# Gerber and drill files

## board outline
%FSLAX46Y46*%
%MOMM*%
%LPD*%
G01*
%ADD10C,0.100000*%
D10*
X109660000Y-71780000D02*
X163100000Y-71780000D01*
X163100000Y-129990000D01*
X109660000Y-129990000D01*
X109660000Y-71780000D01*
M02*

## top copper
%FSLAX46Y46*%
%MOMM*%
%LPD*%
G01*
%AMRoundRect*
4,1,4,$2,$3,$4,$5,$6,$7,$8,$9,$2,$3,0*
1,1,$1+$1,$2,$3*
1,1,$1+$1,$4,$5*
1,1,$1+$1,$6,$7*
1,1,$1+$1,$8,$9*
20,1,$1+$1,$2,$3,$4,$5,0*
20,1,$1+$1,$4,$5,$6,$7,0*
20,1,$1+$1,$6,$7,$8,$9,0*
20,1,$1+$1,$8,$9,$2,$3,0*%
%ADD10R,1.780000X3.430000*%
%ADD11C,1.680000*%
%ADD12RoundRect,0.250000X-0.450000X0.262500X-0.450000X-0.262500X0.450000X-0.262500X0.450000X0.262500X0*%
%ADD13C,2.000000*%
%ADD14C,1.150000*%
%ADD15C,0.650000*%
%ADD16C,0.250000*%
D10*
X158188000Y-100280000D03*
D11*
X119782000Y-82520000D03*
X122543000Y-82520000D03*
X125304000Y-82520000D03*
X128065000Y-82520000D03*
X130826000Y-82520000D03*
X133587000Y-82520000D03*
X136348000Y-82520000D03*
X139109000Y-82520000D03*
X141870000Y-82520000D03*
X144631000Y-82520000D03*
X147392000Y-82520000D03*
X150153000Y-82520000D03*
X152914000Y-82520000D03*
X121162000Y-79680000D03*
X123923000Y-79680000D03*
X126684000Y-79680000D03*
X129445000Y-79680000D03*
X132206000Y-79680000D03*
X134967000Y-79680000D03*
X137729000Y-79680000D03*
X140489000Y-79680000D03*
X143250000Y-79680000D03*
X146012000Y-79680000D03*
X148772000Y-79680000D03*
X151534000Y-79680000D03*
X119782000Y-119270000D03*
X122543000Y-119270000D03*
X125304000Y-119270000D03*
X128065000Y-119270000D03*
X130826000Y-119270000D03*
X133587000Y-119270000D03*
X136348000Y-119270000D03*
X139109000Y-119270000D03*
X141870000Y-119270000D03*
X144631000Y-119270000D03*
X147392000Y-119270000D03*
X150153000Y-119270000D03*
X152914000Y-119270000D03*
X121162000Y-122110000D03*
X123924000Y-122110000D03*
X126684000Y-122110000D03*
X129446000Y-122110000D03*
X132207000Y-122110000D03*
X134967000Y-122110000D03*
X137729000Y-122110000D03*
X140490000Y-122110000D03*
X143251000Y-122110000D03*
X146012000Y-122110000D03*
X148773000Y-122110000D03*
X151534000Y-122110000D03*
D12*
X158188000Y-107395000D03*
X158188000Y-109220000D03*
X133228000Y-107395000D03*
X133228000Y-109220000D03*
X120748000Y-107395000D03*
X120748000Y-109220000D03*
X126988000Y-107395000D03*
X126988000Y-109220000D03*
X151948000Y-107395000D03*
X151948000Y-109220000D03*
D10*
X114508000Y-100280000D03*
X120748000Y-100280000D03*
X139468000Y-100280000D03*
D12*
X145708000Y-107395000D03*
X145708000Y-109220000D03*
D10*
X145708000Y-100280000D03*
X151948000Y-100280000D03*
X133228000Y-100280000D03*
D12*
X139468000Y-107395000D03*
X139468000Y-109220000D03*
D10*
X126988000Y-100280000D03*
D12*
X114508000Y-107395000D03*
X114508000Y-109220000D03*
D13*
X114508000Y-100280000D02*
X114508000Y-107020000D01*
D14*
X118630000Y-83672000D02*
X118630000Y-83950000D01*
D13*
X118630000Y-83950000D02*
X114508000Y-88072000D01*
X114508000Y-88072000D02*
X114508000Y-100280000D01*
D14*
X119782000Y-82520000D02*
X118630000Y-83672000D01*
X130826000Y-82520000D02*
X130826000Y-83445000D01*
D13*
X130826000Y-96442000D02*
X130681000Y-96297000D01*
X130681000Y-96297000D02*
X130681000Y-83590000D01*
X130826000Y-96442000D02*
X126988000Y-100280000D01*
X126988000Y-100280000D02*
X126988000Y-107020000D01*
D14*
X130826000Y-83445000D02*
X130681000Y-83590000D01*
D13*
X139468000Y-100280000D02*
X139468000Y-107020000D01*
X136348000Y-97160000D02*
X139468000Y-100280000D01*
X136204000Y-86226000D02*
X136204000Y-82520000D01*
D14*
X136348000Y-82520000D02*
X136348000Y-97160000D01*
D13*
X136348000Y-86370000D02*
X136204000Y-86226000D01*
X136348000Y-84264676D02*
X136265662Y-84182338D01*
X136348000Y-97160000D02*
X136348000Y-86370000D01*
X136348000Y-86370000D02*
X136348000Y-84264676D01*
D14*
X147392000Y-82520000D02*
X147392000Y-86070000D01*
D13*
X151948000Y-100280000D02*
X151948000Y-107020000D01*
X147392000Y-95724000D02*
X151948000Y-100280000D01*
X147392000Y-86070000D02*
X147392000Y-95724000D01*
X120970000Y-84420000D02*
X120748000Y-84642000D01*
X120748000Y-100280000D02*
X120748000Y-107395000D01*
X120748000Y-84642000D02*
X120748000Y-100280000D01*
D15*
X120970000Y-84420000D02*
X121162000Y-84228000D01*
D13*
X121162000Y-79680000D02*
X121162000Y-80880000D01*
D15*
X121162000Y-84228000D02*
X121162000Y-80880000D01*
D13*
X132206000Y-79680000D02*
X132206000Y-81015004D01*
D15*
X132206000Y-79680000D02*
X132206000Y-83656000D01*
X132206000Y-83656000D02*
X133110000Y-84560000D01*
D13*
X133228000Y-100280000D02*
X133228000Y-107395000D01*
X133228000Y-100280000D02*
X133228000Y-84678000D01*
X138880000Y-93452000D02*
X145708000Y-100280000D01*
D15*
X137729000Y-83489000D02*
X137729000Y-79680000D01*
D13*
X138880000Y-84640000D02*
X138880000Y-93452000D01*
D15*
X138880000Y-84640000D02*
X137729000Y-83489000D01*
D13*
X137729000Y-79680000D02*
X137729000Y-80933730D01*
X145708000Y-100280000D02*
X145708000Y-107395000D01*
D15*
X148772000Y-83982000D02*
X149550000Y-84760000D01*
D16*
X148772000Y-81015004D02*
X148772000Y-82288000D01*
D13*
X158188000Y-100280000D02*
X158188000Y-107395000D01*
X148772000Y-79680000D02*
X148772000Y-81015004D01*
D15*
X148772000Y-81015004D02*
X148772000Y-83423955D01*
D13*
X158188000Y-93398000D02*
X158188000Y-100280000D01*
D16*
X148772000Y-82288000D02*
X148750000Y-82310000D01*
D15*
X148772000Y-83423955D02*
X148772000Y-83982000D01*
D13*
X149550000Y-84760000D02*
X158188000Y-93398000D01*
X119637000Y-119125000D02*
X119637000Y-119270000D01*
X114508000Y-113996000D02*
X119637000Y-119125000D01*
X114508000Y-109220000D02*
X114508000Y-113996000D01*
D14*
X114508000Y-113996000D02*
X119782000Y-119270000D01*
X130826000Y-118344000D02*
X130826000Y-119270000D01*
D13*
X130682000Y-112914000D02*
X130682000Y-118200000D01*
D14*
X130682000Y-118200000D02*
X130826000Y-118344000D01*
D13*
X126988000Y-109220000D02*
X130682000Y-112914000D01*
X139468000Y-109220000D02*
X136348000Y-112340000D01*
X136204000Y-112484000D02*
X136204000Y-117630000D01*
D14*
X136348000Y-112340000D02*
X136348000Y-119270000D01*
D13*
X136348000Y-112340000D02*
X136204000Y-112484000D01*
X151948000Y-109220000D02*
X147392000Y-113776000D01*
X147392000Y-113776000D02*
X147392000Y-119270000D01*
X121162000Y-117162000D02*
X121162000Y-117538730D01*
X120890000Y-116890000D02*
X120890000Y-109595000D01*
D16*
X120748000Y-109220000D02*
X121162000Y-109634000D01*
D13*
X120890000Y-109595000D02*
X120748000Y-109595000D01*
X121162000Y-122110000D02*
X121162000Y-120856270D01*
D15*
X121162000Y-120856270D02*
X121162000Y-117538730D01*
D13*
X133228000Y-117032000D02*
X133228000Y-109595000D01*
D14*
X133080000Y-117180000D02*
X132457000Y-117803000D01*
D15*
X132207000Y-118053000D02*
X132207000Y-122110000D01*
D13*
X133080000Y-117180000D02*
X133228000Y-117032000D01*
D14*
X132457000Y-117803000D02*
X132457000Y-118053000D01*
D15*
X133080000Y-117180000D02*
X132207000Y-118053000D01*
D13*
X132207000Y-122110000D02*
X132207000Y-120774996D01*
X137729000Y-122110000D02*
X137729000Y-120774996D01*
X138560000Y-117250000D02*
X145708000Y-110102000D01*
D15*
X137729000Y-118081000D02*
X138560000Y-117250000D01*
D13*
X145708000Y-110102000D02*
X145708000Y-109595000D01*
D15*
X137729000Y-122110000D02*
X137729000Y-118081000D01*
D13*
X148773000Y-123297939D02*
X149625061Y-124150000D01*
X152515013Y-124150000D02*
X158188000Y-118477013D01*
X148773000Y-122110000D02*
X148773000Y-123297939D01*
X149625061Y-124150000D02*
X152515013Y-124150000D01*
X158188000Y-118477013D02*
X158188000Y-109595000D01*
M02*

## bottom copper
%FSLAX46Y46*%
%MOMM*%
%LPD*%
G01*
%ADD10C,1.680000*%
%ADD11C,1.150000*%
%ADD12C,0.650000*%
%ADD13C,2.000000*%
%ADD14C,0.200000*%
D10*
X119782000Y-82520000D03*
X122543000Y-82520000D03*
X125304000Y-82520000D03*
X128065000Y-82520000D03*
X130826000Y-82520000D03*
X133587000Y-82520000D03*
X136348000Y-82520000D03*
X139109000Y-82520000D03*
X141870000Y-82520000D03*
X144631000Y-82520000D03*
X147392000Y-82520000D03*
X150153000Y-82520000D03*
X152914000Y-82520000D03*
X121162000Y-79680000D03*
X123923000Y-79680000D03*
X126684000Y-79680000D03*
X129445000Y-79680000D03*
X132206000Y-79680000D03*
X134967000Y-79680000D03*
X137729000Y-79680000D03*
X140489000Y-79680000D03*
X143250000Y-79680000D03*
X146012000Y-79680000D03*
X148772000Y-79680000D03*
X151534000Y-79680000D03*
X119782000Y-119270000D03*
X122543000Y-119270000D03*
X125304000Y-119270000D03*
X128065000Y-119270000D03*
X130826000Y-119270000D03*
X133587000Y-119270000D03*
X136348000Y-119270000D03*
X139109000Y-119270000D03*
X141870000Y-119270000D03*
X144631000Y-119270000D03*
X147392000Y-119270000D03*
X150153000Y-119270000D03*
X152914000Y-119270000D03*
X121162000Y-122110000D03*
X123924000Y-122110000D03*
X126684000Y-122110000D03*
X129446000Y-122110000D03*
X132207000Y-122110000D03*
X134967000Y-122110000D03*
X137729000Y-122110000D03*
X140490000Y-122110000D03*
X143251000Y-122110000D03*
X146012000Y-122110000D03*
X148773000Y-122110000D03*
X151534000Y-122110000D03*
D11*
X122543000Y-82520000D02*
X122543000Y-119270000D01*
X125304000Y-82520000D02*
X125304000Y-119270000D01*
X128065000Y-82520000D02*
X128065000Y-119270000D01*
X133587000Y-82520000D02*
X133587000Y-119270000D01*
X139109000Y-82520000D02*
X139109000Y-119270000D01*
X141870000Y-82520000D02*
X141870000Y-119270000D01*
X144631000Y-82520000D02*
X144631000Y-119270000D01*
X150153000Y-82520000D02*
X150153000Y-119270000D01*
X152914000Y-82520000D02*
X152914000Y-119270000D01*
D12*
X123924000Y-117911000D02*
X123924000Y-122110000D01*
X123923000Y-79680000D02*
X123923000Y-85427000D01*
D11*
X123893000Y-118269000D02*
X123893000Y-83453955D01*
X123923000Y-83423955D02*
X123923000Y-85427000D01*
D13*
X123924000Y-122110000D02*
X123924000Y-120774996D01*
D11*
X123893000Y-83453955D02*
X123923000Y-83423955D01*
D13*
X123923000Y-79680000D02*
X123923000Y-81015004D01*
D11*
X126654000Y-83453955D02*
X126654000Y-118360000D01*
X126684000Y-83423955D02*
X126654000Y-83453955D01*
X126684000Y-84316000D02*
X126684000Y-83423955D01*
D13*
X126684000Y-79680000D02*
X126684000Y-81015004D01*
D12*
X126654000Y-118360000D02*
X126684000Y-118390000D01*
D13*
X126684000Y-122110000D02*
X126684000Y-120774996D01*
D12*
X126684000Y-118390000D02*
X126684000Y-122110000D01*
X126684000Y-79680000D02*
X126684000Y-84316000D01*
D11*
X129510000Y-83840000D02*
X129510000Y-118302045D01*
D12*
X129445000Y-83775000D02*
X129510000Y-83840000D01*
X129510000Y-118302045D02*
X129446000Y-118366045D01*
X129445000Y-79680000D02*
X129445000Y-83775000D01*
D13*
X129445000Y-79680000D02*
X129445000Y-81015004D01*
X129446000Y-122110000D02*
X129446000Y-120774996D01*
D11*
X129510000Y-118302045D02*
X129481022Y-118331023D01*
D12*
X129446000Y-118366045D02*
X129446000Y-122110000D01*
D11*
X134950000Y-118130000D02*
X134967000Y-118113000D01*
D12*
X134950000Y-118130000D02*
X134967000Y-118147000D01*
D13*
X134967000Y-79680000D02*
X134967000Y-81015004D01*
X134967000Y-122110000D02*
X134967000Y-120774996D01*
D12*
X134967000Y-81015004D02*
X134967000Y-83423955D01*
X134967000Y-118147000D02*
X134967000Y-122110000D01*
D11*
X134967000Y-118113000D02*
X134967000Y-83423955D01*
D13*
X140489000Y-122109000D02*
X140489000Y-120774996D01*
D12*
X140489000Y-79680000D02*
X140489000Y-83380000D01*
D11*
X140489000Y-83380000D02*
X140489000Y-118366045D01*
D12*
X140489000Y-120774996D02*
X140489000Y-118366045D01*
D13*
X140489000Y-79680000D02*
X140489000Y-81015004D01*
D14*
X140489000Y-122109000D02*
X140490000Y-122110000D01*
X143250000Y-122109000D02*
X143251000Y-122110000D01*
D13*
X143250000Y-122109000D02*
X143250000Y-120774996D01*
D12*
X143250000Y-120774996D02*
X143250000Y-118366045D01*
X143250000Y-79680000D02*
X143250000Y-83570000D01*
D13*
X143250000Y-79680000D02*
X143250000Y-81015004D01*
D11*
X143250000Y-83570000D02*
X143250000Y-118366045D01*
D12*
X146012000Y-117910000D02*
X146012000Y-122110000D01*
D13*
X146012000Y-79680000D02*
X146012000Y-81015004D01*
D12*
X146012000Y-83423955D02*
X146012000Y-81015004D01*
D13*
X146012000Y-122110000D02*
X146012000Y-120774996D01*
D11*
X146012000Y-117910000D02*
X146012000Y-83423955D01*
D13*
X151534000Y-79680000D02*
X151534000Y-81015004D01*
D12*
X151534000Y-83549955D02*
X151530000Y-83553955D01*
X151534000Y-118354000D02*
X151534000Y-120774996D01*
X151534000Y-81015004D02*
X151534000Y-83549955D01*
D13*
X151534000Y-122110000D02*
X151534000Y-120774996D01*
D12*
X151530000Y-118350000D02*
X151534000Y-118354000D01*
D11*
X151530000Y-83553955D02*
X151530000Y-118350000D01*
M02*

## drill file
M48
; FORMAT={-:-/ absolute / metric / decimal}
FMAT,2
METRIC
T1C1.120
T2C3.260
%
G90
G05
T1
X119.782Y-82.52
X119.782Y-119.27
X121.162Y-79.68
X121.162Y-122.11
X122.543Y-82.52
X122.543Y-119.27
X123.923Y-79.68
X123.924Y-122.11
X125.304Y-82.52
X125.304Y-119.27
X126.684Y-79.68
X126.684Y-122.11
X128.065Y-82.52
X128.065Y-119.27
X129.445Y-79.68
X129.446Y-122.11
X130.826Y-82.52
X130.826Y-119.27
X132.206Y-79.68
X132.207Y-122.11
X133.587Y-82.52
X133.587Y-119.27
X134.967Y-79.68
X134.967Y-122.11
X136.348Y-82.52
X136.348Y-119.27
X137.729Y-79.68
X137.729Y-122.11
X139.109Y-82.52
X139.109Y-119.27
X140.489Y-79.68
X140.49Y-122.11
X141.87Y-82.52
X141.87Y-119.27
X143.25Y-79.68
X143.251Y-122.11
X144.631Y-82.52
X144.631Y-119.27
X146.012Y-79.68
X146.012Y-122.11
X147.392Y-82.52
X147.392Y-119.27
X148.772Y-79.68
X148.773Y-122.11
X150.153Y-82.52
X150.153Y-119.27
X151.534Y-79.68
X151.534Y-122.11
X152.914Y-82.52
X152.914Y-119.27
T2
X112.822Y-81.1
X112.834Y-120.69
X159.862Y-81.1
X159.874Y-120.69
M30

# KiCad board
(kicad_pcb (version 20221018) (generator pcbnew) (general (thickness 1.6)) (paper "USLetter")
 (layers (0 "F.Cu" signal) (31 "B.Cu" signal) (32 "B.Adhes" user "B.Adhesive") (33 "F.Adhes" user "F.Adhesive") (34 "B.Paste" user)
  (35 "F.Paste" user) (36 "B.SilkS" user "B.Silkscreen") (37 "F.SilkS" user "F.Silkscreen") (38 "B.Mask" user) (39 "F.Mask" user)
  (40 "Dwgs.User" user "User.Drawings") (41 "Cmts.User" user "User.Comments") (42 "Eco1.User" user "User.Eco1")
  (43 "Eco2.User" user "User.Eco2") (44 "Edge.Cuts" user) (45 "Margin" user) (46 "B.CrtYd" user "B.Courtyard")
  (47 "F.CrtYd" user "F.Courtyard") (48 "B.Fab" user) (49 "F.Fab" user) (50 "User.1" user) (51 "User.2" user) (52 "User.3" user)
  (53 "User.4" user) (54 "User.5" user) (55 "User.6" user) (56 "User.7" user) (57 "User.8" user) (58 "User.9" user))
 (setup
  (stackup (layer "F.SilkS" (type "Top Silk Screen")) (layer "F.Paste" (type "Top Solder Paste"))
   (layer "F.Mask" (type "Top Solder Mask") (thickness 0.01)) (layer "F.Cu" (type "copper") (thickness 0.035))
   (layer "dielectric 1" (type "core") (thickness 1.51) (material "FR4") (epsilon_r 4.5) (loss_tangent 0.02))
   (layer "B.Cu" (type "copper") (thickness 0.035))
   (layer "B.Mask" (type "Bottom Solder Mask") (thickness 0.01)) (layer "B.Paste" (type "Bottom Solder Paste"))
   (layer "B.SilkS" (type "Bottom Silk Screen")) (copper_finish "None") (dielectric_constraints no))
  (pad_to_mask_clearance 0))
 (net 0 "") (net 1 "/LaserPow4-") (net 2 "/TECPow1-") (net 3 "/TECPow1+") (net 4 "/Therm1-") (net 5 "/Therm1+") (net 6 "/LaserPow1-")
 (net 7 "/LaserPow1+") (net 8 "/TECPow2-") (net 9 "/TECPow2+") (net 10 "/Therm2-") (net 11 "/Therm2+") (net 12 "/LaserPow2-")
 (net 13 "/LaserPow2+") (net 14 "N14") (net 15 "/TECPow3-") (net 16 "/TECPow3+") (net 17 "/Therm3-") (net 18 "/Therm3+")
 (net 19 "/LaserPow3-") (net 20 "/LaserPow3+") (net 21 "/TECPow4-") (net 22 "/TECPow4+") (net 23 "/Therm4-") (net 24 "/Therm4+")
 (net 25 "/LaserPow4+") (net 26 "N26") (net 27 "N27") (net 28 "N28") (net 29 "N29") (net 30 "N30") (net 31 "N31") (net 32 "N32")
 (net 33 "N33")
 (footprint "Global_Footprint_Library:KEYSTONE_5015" (layer "F.Cu") (at 158.188 100.28 90)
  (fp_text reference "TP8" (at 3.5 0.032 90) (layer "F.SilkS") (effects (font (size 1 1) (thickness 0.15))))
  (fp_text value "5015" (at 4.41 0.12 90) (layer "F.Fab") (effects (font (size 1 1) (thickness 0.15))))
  (pad "TP" smd rect (at 0 0 90) (size 3.43 1.78) (layers "F.Cu" "F.Paste" "F.Mask") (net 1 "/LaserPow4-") (solder_mask_margin 0.102)))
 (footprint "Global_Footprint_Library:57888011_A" (layer "F.Cu") (at 119.782 82.52)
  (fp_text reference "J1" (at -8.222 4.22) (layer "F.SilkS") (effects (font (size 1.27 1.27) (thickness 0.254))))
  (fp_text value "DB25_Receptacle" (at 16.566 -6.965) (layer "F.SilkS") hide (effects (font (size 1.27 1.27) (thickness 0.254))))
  (pad "" np_thru_hole circle (at -6.96 -1.42) (size 3.26 3.26) (drill 3.26) (layers "*.Cu" "*.Mask"))
  (pad "" np_thru_hole circle (at 40.08 -1.42) (size 3.26 3.26) (drill 3.26) (layers "*.Cu" "*.Mask"))
  (pad "1" thru_hole circle (at 0 0) (size 1.68 1.68) (drill 1.12) (layers "*.Cu" "*.Mask") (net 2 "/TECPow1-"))
  (pad "2" thru_hole circle (at 2.761 0) (size 1.68 1.68) (drill 1.12) (layers "*.Cu" "*.Mask") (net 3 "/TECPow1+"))
  (pad "3" thru_hole circle (at 5.522 0) (size 1.68 1.68) (drill 1.12) (layers "*.Cu" "*.Mask") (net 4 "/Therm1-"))
  (pad "4" thru_hole circle (at 8.283 0) (size 1.68 1.68) (drill 1.12) (layers "*.Cu" "*.Mask") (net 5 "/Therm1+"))
  (pad "5" thru_hole circle (at 11.044 0) (size 1.68 1.68) (drill 1.12) (layers "*.Cu" "*.Mask") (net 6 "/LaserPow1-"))
  (pad "6" thru_hole circle (at 13.805 0) (size 1.68 1.68) (drill 1.12) (layers "*.Cu" "*.Mask") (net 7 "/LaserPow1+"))
  (pad "7" thru_hole circle (at 16.566 0) (size 1.68 1.68) (drill 1.12) (layers "*.Cu" "*.Mask") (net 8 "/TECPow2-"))
  (pad "8" thru_hole circle (at 19.327 0) (size 1.68 1.68) (drill 1.12) (layers "*.Cu" "*.Mask") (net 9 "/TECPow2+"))
  (pad "9" thru_hole circle (at 22.088 0) (size 1.68 1.68) (drill 1.12) (layers "*.Cu" "*.Mask") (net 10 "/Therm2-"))
  (pad "10" thru_hole circle (at 24.849 0) (size 1.68 1.68) (drill 1.12) (layers "*.Cu" "*.Mask") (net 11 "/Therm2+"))
  (pad "11" thru_hole circle (at 27.61 0) (size 1.68 1.68) (drill 1.12) (layers "*.Cu" "*.Mask") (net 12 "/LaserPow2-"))
  (pad "12" thru_hole circle (at 30.371 0) (size 1.68 1.68) (drill 1.12) (layers "*.Cu" "*.Mask") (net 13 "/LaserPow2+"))
  (pad "13" thru_hole circle (at 33.132 0) (size 1.68 1.68) (drill 1.12) (layers "*.Cu" "*.Mask") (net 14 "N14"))
  (pad "14" thru_hole circle (at 1.38 -2.84) (size 1.68 1.68) (drill 1.12) (layers "*.Cu" "*.Mask") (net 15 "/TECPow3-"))
  (pad "15" thru_hole circle (at 4.141 -2.84) (size 1.68 1.68) (drill 1.12) (layers "*.Cu" "*.Mask") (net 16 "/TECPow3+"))
  (pad "16" thru_hole circle (at 6.902 -2.84) (size 1.68 1.68) (drill 1.12) (layers "*.Cu" "*.Mask") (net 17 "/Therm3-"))
  (pad "17" thru_hole circle (at 9.663 -2.84) (size 1.68 1.68) (drill 1.12) (layers "*.Cu" "*.Mask") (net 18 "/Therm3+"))
  (pad "18" thru_hole circle (at 12.424 -2.84) (size 1.68 1.68) (drill 1.12) (layers "*.Cu" "*.Mask") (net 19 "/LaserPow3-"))
  (pad "19" thru_hole circle (at 15.185 -2.84) (size 1.68 1.68) (drill 1.12) (layers "*.Cu" "*.Mask") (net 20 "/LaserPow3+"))
  (pad "20" thru_hole circle (at 17.947 -2.84) (size 1.68 1.68) (drill 1.12) (layers "*.Cu" "*.Mask") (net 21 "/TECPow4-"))
  (pad "21" thru_hole circle (at 20.707 -2.84) (size 1.68 1.68) (drill 1.12) (layers "*.Cu" "*.Mask") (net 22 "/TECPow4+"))
  (pad "22" thru_hole circle (at 23.468 -2.84) (size 1.68 1.68) (drill 1.12) (layers "*.Cu" "*.Mask") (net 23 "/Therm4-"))
  (pad "23" thru_hole circle (at 26.23 -2.84) (size 1.68 1.68) (drill 1.12) (layers "*.Cu" "*.Mask") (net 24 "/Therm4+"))
  (pad "24" thru_hole circle (at 28.99 -2.84) (size 1.68 1.68) (drill 1.12) (layers "*.Cu" "*.Mask") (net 1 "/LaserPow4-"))
  (pad "25" thru_hole circle (at 31.752 -2.84) (size 1.68 1.68) (drill 1.12) (layers "*.Cu" "*.Mask") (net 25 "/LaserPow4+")))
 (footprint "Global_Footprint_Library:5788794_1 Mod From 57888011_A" (layer "F.Cu") (at 152.914 119.27 180)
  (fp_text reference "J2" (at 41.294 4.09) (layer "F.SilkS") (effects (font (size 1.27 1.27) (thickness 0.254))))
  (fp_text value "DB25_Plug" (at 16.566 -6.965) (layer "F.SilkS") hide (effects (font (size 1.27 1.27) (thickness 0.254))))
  (pad "" np_thru_hole circle (at -6.96 -1.42 180) (size 3.26 3.26) (drill 3.26) (layers "*.Cu" "*.Mask"))
  (pad "" np_thru_hole circle (at 40.08 -1.42 180) (size 3.26 3.26) (drill 3.26) (layers "*.Cu" "*.Mask"))
  (pad "1" thru_hole circle (at 33.132 0 180) (size 1.68 1.68) (drill 1.12) (layers "*.Cu" "*.Mask") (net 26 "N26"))
  (pad "2" thru_hole circle (at 30.371 0 180) (size 1.68 1.68) (drill 1.12) (layers "*.Cu" "*.Mask") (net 3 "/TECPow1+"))
  (pad "3" thru_hole circle (at 27.61 0 180) (size 1.68 1.68) (drill 1.12) (layers "*.Cu" "*.Mask") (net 4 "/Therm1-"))
  (pad "4" thru_hole circle (at 24.849 0 180) (size 1.68 1.68) (drill 1.12) (layers "*.Cu" "*.Mask") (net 5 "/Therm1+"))
  (pad "5" thru_hole circle (at 22.088 0 180) (size 1.68 1.68) (drill 1.12) (layers "*.Cu" "*.Mask") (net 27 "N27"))
  (pad "6" thru_hole circle (at 19.327 0 180) (size 1.68 1.68) (drill 1.12) (layers "*.Cu" "*.Mask") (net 7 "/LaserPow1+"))
  (pad "7" thru_hole circle (at 16.566 0 180) (size 1.68 1.68) (drill 1.12) (layers "*.Cu" "*.Mask") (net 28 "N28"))
  (pad "8" thru_hole circle (at 13.805 0 180) (size 1.68 1.68) (drill 1.12) (layers "*.Cu" "*.Mask") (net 9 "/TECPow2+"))
  (pad "9" thru_hole circle (at 11.044 0 180) (size 1.68 1.68) (drill 1.12) (layers "*.Cu" "*.Mask") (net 10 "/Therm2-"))
  (pad "10" thru_hole circle (at 8.283 0 180) (size 1.68 1.68) (drill 1.12) (layers "*.Cu" "*.Mask") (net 11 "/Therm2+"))
  (pad "11" thru_hole circle (at 5.522 0 180) (size 1.68 1.68) (drill 1.12) (layers "*.Cu" "*.Mask") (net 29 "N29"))
  (pad "12" thru_hole circle (at 2.761 0 180) (size 1.68 1.68) (drill 1.12) (layers "*.Cu" "*.Mask") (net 13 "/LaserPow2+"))
  (pad "13" thru_hole circle (at 0 0 180) (size 1.68 1.68) (drill 1.12) (layers "*.Cu" "*.Mask") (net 14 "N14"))
  (pad "14" thru_hole circle (at 31.752 -2.84 180) (size 1.68 1.68) (drill 1.12) (layers "*.Cu" "*.Mask") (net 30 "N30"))
  (pad "15" thru_hole circle (at 28.99 -2.84 180) (size 1.68 1.68) (drill 1.12) (layers "*.Cu" "*.Mask") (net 16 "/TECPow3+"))
  (pad "16" thru_hole circle (at 26.23 -2.84 180) (size 1.68 1.68) (drill 1.12) (layers "*.Cu" "*.Mask") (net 17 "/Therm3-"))
  (pad "17" thru_hole circle (at 23.468 -2.84 180) (size 1.68 1.68) (drill 1.12) (layers "*.Cu" "*.Mask") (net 18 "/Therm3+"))
  (pad "18" thru_hole circle (at 20.707 -2.84 180) (size 1.68 1.68) (drill 1.12) (layers "*.Cu" "*.Mask") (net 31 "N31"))
  (pad "19" thru_hole circle (at 17.947 -2.84 180) (size 1.68 1.68) (drill 1.12) (layers "*.Cu" "*.Mask") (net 20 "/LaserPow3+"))
  (pad "20" thru_hole circle (at 15.185 -2.84 180) (size 1.68 1.68) (drill 1.12) (layers "*.Cu" "*.Mask") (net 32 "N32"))
  (pad "21" thru_hole circle (at 12.424 -2.84 180) (size 1.68 1.68) (drill 1.12) (layers "*.Cu" "*.Mask") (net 22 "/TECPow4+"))
  (pad "22" thru_hole circle (at 9.663 -2.84 180) (size 1.68 1.68) (drill 1.12) (layers "*.Cu" "*.Mask") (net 23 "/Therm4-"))
  (pad "23" thru_hole circle (at 6.902 -2.84 180) (size 1.68 1.68) (drill 1.12) (layers "*.Cu" "*.Mask") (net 24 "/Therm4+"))
  (pad "24" thru_hole circle (at 4.141 -2.84 180) (size 1.68 1.68) (drill 1.12) (layers "*.Cu" "*.Mask") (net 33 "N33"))
  (pad "25" thru_hole circle (at 1.38 -2.84 180) (size 1.68 1.68) (drill 1.12) (layers "*.Cu" "*.Mask") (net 25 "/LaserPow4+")))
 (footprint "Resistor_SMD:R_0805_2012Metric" (layer "F.Cu") (at 158.188 108.3075 -90)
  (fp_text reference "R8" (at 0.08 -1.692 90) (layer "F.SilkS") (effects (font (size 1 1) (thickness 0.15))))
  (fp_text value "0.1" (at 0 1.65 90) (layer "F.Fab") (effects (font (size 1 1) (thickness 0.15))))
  (pad "1" smd roundrect (at -0.9125 0 270) (size 1.025 1.4) (layers "F.Cu" "F.Paste" "F.Mask") (roundrect_rratio 0.243902439)
   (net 1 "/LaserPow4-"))
  (pad "2" smd roundrect (at 0.9125 0 270) (size 1.025 1.4) (layers "F.Cu" "F.Paste" "F.Mask") (roundrect_rratio 0.243902439) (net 33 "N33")))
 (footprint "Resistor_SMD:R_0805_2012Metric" (layer "F.Cu") (at 133.228 108.3075 -90)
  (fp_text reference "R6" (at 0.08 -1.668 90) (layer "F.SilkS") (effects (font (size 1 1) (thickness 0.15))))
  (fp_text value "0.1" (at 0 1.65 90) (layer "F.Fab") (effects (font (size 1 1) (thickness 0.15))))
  (pad "1" smd roundrect (at -0.9125 0 270) (size 1.025 1.4) (layers "F.Cu" "F.Paste" "F.Mask") (roundrect_rratio 0.243902439)
   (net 19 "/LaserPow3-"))
  (pad "2" smd roundrect (at 0.9125 0 270) (size 1.025 1.4) (layers "F.Cu" "F.Paste" "F.Mask") (roundrect_rratio 0.243902439) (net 31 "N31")))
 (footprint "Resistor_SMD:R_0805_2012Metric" (layer "F.Cu") (at 120.748 108.3075 -90)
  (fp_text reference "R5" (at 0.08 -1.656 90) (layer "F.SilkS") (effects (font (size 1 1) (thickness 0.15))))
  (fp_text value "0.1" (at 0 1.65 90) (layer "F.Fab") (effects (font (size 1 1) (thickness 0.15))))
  (pad "1" smd roundrect (at -0.9125 0 270) (size 1.025 1.4) (layers "F.Cu" "F.Paste" "F.Mask") (roundrect_rratio 0.243902439)
   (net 15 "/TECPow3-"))
  (pad "2" smd roundrect (at 0.9125 0 270) (size 1.025 1.4) (layers "F.Cu" "F.Paste" "F.Mask") (roundrect_rratio 0.243902439) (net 30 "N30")))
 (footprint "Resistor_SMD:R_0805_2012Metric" (layer "F.Cu") (at 126.988 108.3075 -90)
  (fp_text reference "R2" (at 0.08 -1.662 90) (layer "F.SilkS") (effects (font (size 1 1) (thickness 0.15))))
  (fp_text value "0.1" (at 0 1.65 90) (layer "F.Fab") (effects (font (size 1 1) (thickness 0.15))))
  (pad "1" smd roundrect (at -0.9125 0 270) (size 1.025 1.4) (layers "F.Cu" "F.Paste" "F.Mask") (roundrect_rratio 0.243902439)
   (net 6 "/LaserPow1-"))
  (pad "2" smd roundrect (at 0.9125 0 270) (size 1.025 1.4) (layers "F.Cu" "F.Paste" "F.Mask") (roundrect_rratio 0.243902439) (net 27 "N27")))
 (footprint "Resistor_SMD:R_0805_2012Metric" (layer "F.Cu") (at 151.948 108.3075 -90)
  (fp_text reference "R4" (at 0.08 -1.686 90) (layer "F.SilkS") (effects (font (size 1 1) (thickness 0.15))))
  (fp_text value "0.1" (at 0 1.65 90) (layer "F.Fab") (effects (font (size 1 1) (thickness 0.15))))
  (pad "1" smd roundrect (at -0.9125 0 270) (size 1.025 1.4) (layers "F.Cu" "F.Paste" "F.Mask") (roundrect_rratio 0.243902439)
   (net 12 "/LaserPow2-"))
  (pad "2" smd roundrect (at 0.9125 0 270) (size 1.025 1.4) (layers "F.Cu" "F.Paste" "F.Mask") (roundrect_rratio 0.243902439) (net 29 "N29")))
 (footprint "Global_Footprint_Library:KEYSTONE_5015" (layer "F.Cu") (at 114.508 100.28 90)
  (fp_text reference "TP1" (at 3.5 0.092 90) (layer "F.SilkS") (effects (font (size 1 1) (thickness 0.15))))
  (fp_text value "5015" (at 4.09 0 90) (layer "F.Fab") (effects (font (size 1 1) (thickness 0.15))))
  (pad "TP" smd rect (at 0 0 90) (size 3.43 1.78) (layers "F.Cu" "F.Paste" "F.Mask") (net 2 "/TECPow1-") (solder_mask_margin 0.102)))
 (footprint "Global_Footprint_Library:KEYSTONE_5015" (layer "F.Cu") (at 120.748 100.28 90)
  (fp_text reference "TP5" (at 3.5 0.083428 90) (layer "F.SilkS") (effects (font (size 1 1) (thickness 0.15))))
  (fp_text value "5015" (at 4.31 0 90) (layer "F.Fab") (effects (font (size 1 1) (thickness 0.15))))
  (pad "TP" smd rect (at 0 0 90) (size 3.43 1.78) (layers "F.Cu" "F.Paste" "F.Mask") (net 15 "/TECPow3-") (solder_mask_margin 0.102)))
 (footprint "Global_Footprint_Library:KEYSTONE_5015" (layer "F.Cu") (at 139.468 100.28 90)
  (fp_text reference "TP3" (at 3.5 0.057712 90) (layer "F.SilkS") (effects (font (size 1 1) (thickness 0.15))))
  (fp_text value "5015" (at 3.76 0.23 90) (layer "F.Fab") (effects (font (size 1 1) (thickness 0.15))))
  (pad "TP" smd rect (at 0 0 90) (size 3.43 1.78) (layers "F.Cu" "F.Paste" "F.Mask") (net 8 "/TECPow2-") (solder_mask_margin 0.102)))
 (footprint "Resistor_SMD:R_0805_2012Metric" (layer "F.Cu") (at 145.708 108.3075 -90)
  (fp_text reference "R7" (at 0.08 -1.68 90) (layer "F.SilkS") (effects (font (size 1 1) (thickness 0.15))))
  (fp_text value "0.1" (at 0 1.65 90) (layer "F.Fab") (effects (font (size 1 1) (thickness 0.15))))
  (pad "1" smd roundrect (at -0.9125 0 270) (size 1.025 1.4) (layers "F.Cu" "F.Paste" "F.Mask") (roundrect_rratio 0.243902439)
   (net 21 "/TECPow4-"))
  (pad "2" smd roundrect (at 0.9125 0 270) (size 1.025 1.4) (layers "F.Cu" "F.Paste" "F.Mask") (roundrect_rratio 0.243902439) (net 32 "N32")))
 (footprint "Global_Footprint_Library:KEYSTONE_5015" (layer "F.Cu") (at 145.708 100.28 90)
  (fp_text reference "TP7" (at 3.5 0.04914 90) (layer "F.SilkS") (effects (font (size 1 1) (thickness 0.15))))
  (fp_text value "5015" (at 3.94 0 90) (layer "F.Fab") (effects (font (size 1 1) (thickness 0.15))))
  (pad "TP" smd rect (at 0 0 90) (size 3.43 1.78) (layers "F.Cu" "F.Paste" "F.Mask") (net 21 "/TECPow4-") (solder_mask_margin 0.102)))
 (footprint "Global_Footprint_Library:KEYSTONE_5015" (layer "F.Cu") (at 151.948 100.28 90)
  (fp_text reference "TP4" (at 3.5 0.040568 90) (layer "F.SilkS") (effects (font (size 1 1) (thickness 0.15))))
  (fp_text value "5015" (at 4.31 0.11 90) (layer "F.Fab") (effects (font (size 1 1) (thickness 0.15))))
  (pad "TP" smd rect (at 0 0 90) (size 3.43 1.78) (layers "F.Cu" "F.Paste" "F.Mask") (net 12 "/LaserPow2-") (solder_mask_margin 0.102)))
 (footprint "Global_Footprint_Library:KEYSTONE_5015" (layer "F.Cu") (at 133.228 100.28 90)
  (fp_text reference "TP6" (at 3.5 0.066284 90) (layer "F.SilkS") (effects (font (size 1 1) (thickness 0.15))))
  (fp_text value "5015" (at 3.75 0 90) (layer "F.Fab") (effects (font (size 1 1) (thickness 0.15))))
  (pad "TP" smd rect (at 0 0 90) (size 3.43 1.78) (layers "F.Cu" "F.Paste" "F.Mask") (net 19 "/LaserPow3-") (solder_mask_margin 0.102)))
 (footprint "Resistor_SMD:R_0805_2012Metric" (layer "F.Cu") (at 139.468 108.3075 -90)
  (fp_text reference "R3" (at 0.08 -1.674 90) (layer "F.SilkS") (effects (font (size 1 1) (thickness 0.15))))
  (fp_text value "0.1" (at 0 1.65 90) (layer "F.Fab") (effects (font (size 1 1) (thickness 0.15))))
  (pad "1" smd roundrect (at -0.9125 0 270) (size 1.025 1.4) (layers "F.Cu" "F.Paste" "F.Mask") (roundrect_rratio 0.243902439)
   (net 8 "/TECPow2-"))
  (pad "2" smd roundrect (at 0.9125 0 270) (size 1.025 1.4) (layers "F.Cu" "F.Paste" "F.Mask") (roundrect_rratio 0.243902439) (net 28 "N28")))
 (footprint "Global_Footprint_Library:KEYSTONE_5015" (layer "F.Cu") (at 126.988 100.28 90)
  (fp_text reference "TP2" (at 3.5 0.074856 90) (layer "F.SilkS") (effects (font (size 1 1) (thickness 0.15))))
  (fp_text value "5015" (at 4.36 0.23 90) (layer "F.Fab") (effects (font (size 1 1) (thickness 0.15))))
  (pad "TP" smd rect (at 0 0 90) (size 3.43 1.78) (layers "F.Cu" "F.Paste" "F.Mask") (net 6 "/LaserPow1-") (solder_mask_margin 0.102)))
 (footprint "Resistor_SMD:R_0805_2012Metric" (layer "F.Cu") (at 114.508 108.3075 -90)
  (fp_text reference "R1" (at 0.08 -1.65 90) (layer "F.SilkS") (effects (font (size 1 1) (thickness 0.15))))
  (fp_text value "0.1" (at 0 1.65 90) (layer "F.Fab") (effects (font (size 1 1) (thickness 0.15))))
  (pad "1" smd roundrect (at -0.9125 0 270) (size 1.025 1.4) (layers "F.Cu" "F.Paste" "F.Mask") (roundrect_rratio 0.243902439)
   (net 2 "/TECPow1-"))
  (pad "2" smd roundrect (at 0.9125 0 270) (size 1.025 1.4) (layers "F.Cu" "F.Paste" "F.Mask") (roundrect_rratio 0.243902439) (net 26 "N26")))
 (gr_rect (start 109.66 71.78) (end 163.1 129.99) (stroke (width 0.1) (type default)) (fill none) (layer "Edge.Cuts"))
 (segment (start 114.508 100.28) (end 114.508 107.02) (width 2) (layer "F.Cu") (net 2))
 (segment (start 118.63 83.672) (end 118.63 83.95) (width 1.15) (layer "F.Cu") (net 2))
 (segment (start 118.63 83.95) (end 114.508 88.072) (width 2) (layer "F.Cu") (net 2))
 (segment (start 114.508 88.072) (end 114.508 100.28) (width 2) (layer "F.Cu") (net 2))
 (segment (start 119.782 82.52) (end 118.63 83.672) (width 1.15) (layer "F.Cu") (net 2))
 (segment (start 122.543 82.52) (end 122.543 119.27) (width 1.15) (layer "B.Cu") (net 3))
 (segment (start 125.304 82.52) (end 125.304 119.27) (width 1.15) (layer "B.Cu") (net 4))
 (segment (start 128.065 82.52) (end 128.065 119.27) (width 1.15) (layer "B.Cu") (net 5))
 (segment (start 130.826 82.52) (end 130.826 83.445) (width 1.15) (layer "F.Cu") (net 6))
 (segment (start 130.826 96.442) (end 130.681 96.297) (width 2) (layer "F.Cu") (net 6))
 (segment (start 130.681 96.297) (end 130.681 83.59) (width 2) (layer "F.Cu") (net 6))
 (segment (start 130.826 96.442) (end 126.988 100.28) (width 2) (layer "F.Cu") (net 6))
 (segment (start 126.988 100.28) (end 126.988 107.02) (width 2) (layer "F.Cu") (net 6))
 (segment (start 130.826 83.445) (end 130.681 83.59) (width 1.15) (layer "F.Cu") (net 6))
 (segment (start 133.587 82.52) (end 133.587 119.27) (width 1.15) (layer "B.Cu") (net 7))
 (segment (start 139.468 100.28) (end 139.468 107.02) (width 2) (layer "F.Cu") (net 8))
 (segment (start 136.348 97.16) (end 139.468 100.28) (width 2) (layer "F.Cu") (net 8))
 (segment (start 136.204 86.226) (end 136.204 82.52) (width 2) (layer "F.Cu") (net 8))
 (segment (start 136.348 82.52) (end 136.348 97.16) (width 1.15) (layer "F.Cu") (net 8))
 (segment (start 136.348 86.37) (end 136.204 86.226) (width 2) (layer "F.Cu") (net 8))
 (segment (start 136.348 84.264676) (end 136.265662 84.182338) (width 2) (layer "F.Cu") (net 8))
 (segment (start 136.348 97.16) (end 136.348 86.37) (width 2) (layer "F.Cu") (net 8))
 (segment (start 136.348 86.37) (end 136.348 84.264676) (width 2) (layer "F.Cu") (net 8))
 (segment (start 139.109 82.52) (end 139.109 119.27) (width 1.15) (layer "B.Cu") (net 9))
 (segment (start 141.87 82.52) (end 141.87 119.27) (width 1.15) (layer "B.Cu") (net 10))
 (segment (start 144.631 82.52) (end 144.631 119.27) (width 1.15) (layer "B.Cu") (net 11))
 (segment (start 147.392 82.52) (end 147.392 86.07) (width 1.15) (layer "F.Cu") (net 12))
 (segment (start 151.948 100.28) (end 151.948 107.02) (width 2) (layer "F.Cu") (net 12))
 (segment (start 147.392 95.724) (end 151.948 100.28) (width 2) (layer "F.Cu") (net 12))
 (segment (start 147.392 86.07) (end 147.392 95.724) (width 2) (layer "F.Cu") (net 12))
 (segment (start 150.153 82.52) (end 150.153 119.27) (width 1.15) (layer "B.Cu") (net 13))
 (segment (start 152.914 82.52) (end 152.914 119.27) (width 1.15) (layer "B.Cu") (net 14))
 (segment (start 120.97 84.42) (end 120.748 84.642) (width 2) (layer "F.Cu") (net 15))
 (segment (start 120.748 100.28) (end 120.748 107.395) (width 2) (layer "F.Cu") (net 15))
 (segment (start 120.748 84.642) (end 120.748 100.28) (width 2) (layer "F.Cu") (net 15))
 (segment (start 120.97 84.42) (end 121.162 84.228) (width 0.65) (layer "F.Cu") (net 15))
 (segment (start 121.162 79.68) (end 121.162 80.88) (width 2) (layer "F.Cu") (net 15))
 (segment (start 121.162 84.228) (end 121.162 80.88) (width 0.65) (layer "F.Cu") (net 15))
 (segment (start 123.924 117.911) (end 123.924 122.11) (width 0.65) (layer "B.Cu") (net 16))
 (segment (start 123.923 79.68) (end 123.923 85.427) (width 0.65) (layer "B.Cu") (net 16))
 (segment (start 123.893 118.269) (end 123.893 83.453955) (width 1.15) (layer "B.Cu") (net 16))
 (segment (start 123.923 83.423955) (end 123.923 85.427) (width 1.15) (layer "B.Cu") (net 16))
 (segment (start 123.924 122.11) (end 123.924 120.774996) (width 2) (layer "B.Cu") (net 16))
 (segment (start 123.893 83.453955) (end 123.923 83.423955) (width 1.15) (layer "B.Cu") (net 16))
 (segment (start 123.923 79.68) (end 123.923 81.015004) (width 2) (layer "B.Cu") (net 16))
 (segment (start 126.654 83.453955) (end 126.654 118.36) (width 1.15) (layer "B.Cu") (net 17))
 (segment (start 126.684 83.423955) (end 126.654 83.453955) (width 1.15) (layer "B.Cu") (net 17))
 (segment (start 126.684 84.316) (end 126.684 83.423955) (width 1.15) (layer "B.Cu") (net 17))
 (segment (start 126.684 79.68) (end 126.684 81.015004) (width 2) (layer "B.Cu") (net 17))
 (segment (start 126.654 118.36) (end 126.684 118.39) (width 0.65) (layer "B.Cu") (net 17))
 (segment (start 126.684 122.11) (end 126.684 120.774996) (width 2) (layer "B.Cu") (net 17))
 (segment (start 126.684 118.39) (end 126.684 122.11) (width 0.65) (layer "B.Cu") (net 17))
 (segment (start 126.684 79.68) (end 126.684 84.316) (width 0.65) (layer "B.Cu") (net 17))
 (segment (start 129.51 83.84) (end 129.51 118.302045) (width 1.15) (layer "B.Cu") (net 18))
 (segment (start 129.445 83.775) (end 129.51 83.84) (width 0.65) (layer "B.Cu") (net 18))
 (segment (start 129.51 118.302045) (end 129.446 118.366045) (width 0.65) (layer "B.Cu") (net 18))
 (segment (start 129.445 79.68) (end 129.445 83.775) (width 0.65) (layer "B.Cu") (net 18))
 (segment (start 129.445 79.68) (end 129.445 81.015004) (width 2) (layer "B.Cu") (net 18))
 (segment (start 129.446 122.11) (end 129.446 120.774996) (width 2) (layer "B.Cu") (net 18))
 (segment (start 129.51 118.302045) (end 129.481022 118.331023) (width 1.15) (layer "B.Cu") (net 18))
 (segment (start 129.446 118.366045) (end 129.446 122.11) (width 0.65) (layer "B.Cu") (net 18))
 (segment (start 132.206 79.68) (end 132.206 81.015004) (width 2) (layer "F.Cu") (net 19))
 (segment (start 132.206 79.68) (end 132.206 83.656) (width 0.65) (layer "F.Cu") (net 19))
 (segment (start 132.206 83.656) (end 133.11 84.56) (width 0.65) (layer "F.Cu") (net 19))
 (segment (start 133.228 100.28) (end 133.228 107.395) (width 2) (layer "F.Cu") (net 19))
 (segment (start 133.228 100.28) (end 133.228 84.678) (width 2) (layer "F.Cu") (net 19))
 (segment (start 134.95 118.13) (end 134.967 118.113) (width 1.15) (layer "B.Cu") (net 20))
 (segment (start 134.95 118.13) (end 134.967 118.147) (width 0.65) (layer "B.Cu") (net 20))
 (segment (start 134.967 79.68) (end 134.967 81.015004) (width 2) (layer "B.Cu") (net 20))
 (segment (start 134.967 122.11) (end 134.967 120.774996) (width 2) (layer "B.Cu") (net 20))
 (segment (start 134.967 81.015004) (end 134.967 83.423955) (width 0.65) (layer "B.Cu") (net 20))
 (segment (start 134.967 118.147) (end 134.967 122.11) (width 0.65) (layer "B.Cu") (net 20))
 (segment (start 134.967 118.113) (end 134.967 83.423955) (width 1.15) (layer "B.Cu") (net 20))
 (segment (start 138.88 93.452) (end 145.708 100.28) (width 2) (layer "F.Cu") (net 21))
 (segment (start 137.729 83.489) (end 137.729 79.68) (width 0.65) (layer "F.Cu") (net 21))
 (segment (start 138.88 84.64) (end 138.88 93.452) (width 2) (layer "F.Cu") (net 21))
 (segment (start 138.88 84.64) (end 137.729 83.489) (width 0.65) (layer "F.Cu") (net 21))
 (segment (start 137.729 79.68) (end 137.729 80.93373) (width 2) (layer "F.Cu") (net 21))
 (segment (start 145.708 100.28) (end 145.708 107.395) (width 2) (layer "F.Cu") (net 21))
 (segment (start 140.489 122.109) (end 140.489 120.774996) (width 2) (layer "B.Cu") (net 22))
 (segment (start 140.489 79.68) (end 140.489 83.38) (width 0.65) (layer "B.Cu") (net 22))
 (segment (start 140.489 83.38) (end 140.489 118.366045) (width 1.15) (layer "B.Cu") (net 22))
 (segment (start 140.489 120.774996) (end 140.489 118.366045) (width 0.65) (layer "B.Cu") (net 22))
 (segment (start 140.489 79.68) (end 140.489 81.015004) (width 2) (layer "B.Cu") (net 22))
 (segment (start 140.489 122.109) (end 140.49 122.11) (width 0.2) (layer "B.Cu") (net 22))
 (segment (start 143.25 122.109) (end 143.251 122.11) (width 0.2) (layer "B.Cu") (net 23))
 (segment (start 143.25 122.109) (end 143.25 120.774996) (width 2) (layer "B.Cu") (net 23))
 (segment (start 143.25 120.774996) (end 143.25 118.366045) (width 0.65) (layer "B.Cu") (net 23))
 (segment (start 143.25 79.68) (end 143.25 83.57) (width 0.65) (layer "B.Cu") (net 23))
 (segment (start 143.25 79.68) (end 143.25 81.015004) (width 2) (layer "B.Cu") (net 23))
 (segment (start 143.25 83.57) (end 143.25 118.366045) (width 1.15) (layer "B.Cu") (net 23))
 (segment (start 146.012 117.91) (end 146.012 122.11) (width 0.65) (layer "B.Cu") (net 24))
 (segment (start 146.012 79.68) (end 146.012 81.015004) (width 2) (layer "B.Cu") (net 24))
 (segment (start 146.012 83.423955) (end 146.012 81.015004) (width 0.65) (layer "B.Cu") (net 24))
 (segment (start 146.012 122.11) (end 146.012 120.774996) (width 2) (layer "B.Cu") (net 24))
 (segment (start 146.012 117.91) (end 146.012 83.423955) (width 1.15) (layer "B.Cu") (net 24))
 (segment (start 148.772 83.982) (end 149.55 84.76) (width 0.65) (layer "F.Cu") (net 1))
 (segment (start 148.772 81.015004) (end 148.772 82.288) (width 0.25) (layer "F.Cu") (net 1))
 (segment (start 158.188 100.28) (end 158.188 107.395) (width 2) (layer "F.Cu") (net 1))
 (segment (start 148.772 79.68) (end 148.772 81.015004) (width 2) (layer "F.Cu") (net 1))
 (segment (start 148.772 81.015004) (end 148.772 83.423955) (width 0.65) (layer "F.Cu") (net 1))
 (segment (start 158.188 93.398) (end 158.188 100.28) (width 2) (layer "F.Cu") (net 1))
 (segment (start 148.772 82.288) (end 148.75 82.31) (width 0.25) (layer "F.Cu") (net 1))
 (segment (start 148.772 83.423955) (end 148.772 83.982) (width 0.65) (layer "F.Cu") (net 1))
 (segment (start 149.55 84.76) (end 158.188 93.398) (width 2) (layer "F.Cu") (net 1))
 (segment (start 151.534 79.68) (end 151.534 81.015004) (width 2) (layer "B.Cu") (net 25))
 (segment (start 151.534 83.549955) (end 151.53 83.553955) (width 0.65) (layer "B.Cu") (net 25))
 (segment (start 151.534 118.354) (end 151.534 120.774996) (width 0.65) (layer "B.Cu") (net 25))
 (segment (start 151.534 81.015004) (end 151.534 83.549955) (width 0.65) (layer "B.Cu") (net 25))
 (segment (start 151.534 122.11) (end 151.534 120.774996) (width 2) (layer "B.Cu") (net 25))
 (segment (start 151.53 118.35) (end 151.534 118.354) (width 0.65) (layer "B.Cu") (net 25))
 (segment (start 151.53 83.553955) (end 151.53 118.35) (width 1.15) (layer "B.Cu") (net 25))
 (segment (start 119.637 119.125) (end 119.637 119.27) (width 2) (layer "F.Cu") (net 26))
 (segment (start 114.508 113.996) (end 119.637 119.125) (width 2) (layer "F.Cu") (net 26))
 (segment (start 114.508 109.22) (end 114.508 113.996) (width 2) (layer "F.Cu") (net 26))
 (segment (start 114.508 113.996) (end 119.782 119.27) (width 1.15) (layer "F.Cu") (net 26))
 (segment (start 130.826 118.344) (end 130.826 119.27) (width 1.15) (layer "F.Cu") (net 27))
 (segment (start 130.682 112.914) (end 130.682 118.2) (width 2) (layer "F.Cu") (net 27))
 (segment (start 130.682 118.2) (end 130.826 118.344) (width 1.15) (layer "F.Cu") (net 27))
 (segment (start 126.988 109.22) (end 130.682 112.914) (width 2) (layer "F.Cu") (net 27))
 (segment (start 139.468 109.22) (end 136.348 112.34) (width 2) (layer "F.Cu") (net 28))
 (segment (start 136.204 112.484) (end 136.204 117.63) (width 2) (layer "F.Cu") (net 28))
 (segment (start 136.348 112.34) (end 136.348 119.27) (width 1.15) (layer "F.Cu") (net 28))
 (segment (start 136.348 112.34) (end 136.204 112.484) (width 2) (layer "F.Cu") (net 28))
 (segment (start 151.948 109.22) (end 147.392 113.776) (width 2) (layer "F.Cu") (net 29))
 (segment (start 147.392 113.776) (end 147.392 119.27) (width 2) (layer "F.Cu") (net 29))
 (segment (start 121.162 117.162) (end 121.162 117.53873) (width 2) (layer "F.Cu") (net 30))
 (segment (start 120.89 116.89) (end 120.89 109.595) (width 2) (layer "F.Cu") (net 30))
 (segment (start 120.748 109.22) (end 121.162 109.634) (width 0.25) (layer "F.Cu") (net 30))
 (segment (start 120.89 109.595) (end 120.748 109.595) (width 2) (layer "F.Cu") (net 30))
 (segment (start 121.162 122.11) (end 121.162 120.85627) (width 2) (layer "F.Cu") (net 30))
 (segment (start 121.162 120.85627) (end 121.162 117.53873) (width 0.65) (layer "F.Cu") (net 30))
 (segment (start 133.228 117.032) (end 133.228 109.595) (width 2) (layer "F.Cu") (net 31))
 (segment (start 133.08 117.18) (end 132.457 117.803) (width 1.15) (layer "F.Cu") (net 31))
 (segment (start 132.207 118.053) (end 132.207 122.11) (width 0.65) (layer "F.Cu") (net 31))
 (segment (start 133.08 117.18) (end 133.228 117.032) (width 2) (layer "F.Cu") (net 31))
 (segment (start 132.457 117.803) (end 132.457 118.053) (width 1.15) (layer "F.Cu") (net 31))
 (segment (start 133.08 117.18) (end 132.207 118.053) (width 0.65) (layer "F.Cu") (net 31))
 (segment (start 132.207 122.11) (end 132.207 120.774996) (width 2) (layer "F.Cu") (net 31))
 (segment (start 137.729 122.11) (end 137.729 120.774996) (width 2) (layer "F.Cu") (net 32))
 (segment (start 138.56 117.25) (end 145.708 110.102) (width 2) (layer "F.Cu") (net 32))
 (segment (start 137.729 118.081) (end 138.56 117.25) (width 0.65) (layer "F.Cu") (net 32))
 (segment (start 145.708 110.102) (end 145.708 109.595) (width 2) (layer "F.Cu") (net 32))
 (segment (start 137.729 122.11) (end 137.729 118.081) (width 0.65) (layer "F.Cu") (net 32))
 (segment (start 148.773 123.297939) (end 149.625061 124.15) (width 2) (layer "F.Cu") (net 33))
 (segment (start 152.515013 124.15) (end 158.188 118.477013) (width 2) (layer "F.Cu") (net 33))
 (segment (start 148.773 122.11) (end 148.773 123.297939) (width 2) (layer "F.Cu") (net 33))
 (segment (start 149.625061 124.15) (end 152.515013 124.15) (width 2) (layer "F.Cu") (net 33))
 (segment (start 158.188 118.477013) (end 158.188 109.595) (width 2) (layer "F.Cu") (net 33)))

